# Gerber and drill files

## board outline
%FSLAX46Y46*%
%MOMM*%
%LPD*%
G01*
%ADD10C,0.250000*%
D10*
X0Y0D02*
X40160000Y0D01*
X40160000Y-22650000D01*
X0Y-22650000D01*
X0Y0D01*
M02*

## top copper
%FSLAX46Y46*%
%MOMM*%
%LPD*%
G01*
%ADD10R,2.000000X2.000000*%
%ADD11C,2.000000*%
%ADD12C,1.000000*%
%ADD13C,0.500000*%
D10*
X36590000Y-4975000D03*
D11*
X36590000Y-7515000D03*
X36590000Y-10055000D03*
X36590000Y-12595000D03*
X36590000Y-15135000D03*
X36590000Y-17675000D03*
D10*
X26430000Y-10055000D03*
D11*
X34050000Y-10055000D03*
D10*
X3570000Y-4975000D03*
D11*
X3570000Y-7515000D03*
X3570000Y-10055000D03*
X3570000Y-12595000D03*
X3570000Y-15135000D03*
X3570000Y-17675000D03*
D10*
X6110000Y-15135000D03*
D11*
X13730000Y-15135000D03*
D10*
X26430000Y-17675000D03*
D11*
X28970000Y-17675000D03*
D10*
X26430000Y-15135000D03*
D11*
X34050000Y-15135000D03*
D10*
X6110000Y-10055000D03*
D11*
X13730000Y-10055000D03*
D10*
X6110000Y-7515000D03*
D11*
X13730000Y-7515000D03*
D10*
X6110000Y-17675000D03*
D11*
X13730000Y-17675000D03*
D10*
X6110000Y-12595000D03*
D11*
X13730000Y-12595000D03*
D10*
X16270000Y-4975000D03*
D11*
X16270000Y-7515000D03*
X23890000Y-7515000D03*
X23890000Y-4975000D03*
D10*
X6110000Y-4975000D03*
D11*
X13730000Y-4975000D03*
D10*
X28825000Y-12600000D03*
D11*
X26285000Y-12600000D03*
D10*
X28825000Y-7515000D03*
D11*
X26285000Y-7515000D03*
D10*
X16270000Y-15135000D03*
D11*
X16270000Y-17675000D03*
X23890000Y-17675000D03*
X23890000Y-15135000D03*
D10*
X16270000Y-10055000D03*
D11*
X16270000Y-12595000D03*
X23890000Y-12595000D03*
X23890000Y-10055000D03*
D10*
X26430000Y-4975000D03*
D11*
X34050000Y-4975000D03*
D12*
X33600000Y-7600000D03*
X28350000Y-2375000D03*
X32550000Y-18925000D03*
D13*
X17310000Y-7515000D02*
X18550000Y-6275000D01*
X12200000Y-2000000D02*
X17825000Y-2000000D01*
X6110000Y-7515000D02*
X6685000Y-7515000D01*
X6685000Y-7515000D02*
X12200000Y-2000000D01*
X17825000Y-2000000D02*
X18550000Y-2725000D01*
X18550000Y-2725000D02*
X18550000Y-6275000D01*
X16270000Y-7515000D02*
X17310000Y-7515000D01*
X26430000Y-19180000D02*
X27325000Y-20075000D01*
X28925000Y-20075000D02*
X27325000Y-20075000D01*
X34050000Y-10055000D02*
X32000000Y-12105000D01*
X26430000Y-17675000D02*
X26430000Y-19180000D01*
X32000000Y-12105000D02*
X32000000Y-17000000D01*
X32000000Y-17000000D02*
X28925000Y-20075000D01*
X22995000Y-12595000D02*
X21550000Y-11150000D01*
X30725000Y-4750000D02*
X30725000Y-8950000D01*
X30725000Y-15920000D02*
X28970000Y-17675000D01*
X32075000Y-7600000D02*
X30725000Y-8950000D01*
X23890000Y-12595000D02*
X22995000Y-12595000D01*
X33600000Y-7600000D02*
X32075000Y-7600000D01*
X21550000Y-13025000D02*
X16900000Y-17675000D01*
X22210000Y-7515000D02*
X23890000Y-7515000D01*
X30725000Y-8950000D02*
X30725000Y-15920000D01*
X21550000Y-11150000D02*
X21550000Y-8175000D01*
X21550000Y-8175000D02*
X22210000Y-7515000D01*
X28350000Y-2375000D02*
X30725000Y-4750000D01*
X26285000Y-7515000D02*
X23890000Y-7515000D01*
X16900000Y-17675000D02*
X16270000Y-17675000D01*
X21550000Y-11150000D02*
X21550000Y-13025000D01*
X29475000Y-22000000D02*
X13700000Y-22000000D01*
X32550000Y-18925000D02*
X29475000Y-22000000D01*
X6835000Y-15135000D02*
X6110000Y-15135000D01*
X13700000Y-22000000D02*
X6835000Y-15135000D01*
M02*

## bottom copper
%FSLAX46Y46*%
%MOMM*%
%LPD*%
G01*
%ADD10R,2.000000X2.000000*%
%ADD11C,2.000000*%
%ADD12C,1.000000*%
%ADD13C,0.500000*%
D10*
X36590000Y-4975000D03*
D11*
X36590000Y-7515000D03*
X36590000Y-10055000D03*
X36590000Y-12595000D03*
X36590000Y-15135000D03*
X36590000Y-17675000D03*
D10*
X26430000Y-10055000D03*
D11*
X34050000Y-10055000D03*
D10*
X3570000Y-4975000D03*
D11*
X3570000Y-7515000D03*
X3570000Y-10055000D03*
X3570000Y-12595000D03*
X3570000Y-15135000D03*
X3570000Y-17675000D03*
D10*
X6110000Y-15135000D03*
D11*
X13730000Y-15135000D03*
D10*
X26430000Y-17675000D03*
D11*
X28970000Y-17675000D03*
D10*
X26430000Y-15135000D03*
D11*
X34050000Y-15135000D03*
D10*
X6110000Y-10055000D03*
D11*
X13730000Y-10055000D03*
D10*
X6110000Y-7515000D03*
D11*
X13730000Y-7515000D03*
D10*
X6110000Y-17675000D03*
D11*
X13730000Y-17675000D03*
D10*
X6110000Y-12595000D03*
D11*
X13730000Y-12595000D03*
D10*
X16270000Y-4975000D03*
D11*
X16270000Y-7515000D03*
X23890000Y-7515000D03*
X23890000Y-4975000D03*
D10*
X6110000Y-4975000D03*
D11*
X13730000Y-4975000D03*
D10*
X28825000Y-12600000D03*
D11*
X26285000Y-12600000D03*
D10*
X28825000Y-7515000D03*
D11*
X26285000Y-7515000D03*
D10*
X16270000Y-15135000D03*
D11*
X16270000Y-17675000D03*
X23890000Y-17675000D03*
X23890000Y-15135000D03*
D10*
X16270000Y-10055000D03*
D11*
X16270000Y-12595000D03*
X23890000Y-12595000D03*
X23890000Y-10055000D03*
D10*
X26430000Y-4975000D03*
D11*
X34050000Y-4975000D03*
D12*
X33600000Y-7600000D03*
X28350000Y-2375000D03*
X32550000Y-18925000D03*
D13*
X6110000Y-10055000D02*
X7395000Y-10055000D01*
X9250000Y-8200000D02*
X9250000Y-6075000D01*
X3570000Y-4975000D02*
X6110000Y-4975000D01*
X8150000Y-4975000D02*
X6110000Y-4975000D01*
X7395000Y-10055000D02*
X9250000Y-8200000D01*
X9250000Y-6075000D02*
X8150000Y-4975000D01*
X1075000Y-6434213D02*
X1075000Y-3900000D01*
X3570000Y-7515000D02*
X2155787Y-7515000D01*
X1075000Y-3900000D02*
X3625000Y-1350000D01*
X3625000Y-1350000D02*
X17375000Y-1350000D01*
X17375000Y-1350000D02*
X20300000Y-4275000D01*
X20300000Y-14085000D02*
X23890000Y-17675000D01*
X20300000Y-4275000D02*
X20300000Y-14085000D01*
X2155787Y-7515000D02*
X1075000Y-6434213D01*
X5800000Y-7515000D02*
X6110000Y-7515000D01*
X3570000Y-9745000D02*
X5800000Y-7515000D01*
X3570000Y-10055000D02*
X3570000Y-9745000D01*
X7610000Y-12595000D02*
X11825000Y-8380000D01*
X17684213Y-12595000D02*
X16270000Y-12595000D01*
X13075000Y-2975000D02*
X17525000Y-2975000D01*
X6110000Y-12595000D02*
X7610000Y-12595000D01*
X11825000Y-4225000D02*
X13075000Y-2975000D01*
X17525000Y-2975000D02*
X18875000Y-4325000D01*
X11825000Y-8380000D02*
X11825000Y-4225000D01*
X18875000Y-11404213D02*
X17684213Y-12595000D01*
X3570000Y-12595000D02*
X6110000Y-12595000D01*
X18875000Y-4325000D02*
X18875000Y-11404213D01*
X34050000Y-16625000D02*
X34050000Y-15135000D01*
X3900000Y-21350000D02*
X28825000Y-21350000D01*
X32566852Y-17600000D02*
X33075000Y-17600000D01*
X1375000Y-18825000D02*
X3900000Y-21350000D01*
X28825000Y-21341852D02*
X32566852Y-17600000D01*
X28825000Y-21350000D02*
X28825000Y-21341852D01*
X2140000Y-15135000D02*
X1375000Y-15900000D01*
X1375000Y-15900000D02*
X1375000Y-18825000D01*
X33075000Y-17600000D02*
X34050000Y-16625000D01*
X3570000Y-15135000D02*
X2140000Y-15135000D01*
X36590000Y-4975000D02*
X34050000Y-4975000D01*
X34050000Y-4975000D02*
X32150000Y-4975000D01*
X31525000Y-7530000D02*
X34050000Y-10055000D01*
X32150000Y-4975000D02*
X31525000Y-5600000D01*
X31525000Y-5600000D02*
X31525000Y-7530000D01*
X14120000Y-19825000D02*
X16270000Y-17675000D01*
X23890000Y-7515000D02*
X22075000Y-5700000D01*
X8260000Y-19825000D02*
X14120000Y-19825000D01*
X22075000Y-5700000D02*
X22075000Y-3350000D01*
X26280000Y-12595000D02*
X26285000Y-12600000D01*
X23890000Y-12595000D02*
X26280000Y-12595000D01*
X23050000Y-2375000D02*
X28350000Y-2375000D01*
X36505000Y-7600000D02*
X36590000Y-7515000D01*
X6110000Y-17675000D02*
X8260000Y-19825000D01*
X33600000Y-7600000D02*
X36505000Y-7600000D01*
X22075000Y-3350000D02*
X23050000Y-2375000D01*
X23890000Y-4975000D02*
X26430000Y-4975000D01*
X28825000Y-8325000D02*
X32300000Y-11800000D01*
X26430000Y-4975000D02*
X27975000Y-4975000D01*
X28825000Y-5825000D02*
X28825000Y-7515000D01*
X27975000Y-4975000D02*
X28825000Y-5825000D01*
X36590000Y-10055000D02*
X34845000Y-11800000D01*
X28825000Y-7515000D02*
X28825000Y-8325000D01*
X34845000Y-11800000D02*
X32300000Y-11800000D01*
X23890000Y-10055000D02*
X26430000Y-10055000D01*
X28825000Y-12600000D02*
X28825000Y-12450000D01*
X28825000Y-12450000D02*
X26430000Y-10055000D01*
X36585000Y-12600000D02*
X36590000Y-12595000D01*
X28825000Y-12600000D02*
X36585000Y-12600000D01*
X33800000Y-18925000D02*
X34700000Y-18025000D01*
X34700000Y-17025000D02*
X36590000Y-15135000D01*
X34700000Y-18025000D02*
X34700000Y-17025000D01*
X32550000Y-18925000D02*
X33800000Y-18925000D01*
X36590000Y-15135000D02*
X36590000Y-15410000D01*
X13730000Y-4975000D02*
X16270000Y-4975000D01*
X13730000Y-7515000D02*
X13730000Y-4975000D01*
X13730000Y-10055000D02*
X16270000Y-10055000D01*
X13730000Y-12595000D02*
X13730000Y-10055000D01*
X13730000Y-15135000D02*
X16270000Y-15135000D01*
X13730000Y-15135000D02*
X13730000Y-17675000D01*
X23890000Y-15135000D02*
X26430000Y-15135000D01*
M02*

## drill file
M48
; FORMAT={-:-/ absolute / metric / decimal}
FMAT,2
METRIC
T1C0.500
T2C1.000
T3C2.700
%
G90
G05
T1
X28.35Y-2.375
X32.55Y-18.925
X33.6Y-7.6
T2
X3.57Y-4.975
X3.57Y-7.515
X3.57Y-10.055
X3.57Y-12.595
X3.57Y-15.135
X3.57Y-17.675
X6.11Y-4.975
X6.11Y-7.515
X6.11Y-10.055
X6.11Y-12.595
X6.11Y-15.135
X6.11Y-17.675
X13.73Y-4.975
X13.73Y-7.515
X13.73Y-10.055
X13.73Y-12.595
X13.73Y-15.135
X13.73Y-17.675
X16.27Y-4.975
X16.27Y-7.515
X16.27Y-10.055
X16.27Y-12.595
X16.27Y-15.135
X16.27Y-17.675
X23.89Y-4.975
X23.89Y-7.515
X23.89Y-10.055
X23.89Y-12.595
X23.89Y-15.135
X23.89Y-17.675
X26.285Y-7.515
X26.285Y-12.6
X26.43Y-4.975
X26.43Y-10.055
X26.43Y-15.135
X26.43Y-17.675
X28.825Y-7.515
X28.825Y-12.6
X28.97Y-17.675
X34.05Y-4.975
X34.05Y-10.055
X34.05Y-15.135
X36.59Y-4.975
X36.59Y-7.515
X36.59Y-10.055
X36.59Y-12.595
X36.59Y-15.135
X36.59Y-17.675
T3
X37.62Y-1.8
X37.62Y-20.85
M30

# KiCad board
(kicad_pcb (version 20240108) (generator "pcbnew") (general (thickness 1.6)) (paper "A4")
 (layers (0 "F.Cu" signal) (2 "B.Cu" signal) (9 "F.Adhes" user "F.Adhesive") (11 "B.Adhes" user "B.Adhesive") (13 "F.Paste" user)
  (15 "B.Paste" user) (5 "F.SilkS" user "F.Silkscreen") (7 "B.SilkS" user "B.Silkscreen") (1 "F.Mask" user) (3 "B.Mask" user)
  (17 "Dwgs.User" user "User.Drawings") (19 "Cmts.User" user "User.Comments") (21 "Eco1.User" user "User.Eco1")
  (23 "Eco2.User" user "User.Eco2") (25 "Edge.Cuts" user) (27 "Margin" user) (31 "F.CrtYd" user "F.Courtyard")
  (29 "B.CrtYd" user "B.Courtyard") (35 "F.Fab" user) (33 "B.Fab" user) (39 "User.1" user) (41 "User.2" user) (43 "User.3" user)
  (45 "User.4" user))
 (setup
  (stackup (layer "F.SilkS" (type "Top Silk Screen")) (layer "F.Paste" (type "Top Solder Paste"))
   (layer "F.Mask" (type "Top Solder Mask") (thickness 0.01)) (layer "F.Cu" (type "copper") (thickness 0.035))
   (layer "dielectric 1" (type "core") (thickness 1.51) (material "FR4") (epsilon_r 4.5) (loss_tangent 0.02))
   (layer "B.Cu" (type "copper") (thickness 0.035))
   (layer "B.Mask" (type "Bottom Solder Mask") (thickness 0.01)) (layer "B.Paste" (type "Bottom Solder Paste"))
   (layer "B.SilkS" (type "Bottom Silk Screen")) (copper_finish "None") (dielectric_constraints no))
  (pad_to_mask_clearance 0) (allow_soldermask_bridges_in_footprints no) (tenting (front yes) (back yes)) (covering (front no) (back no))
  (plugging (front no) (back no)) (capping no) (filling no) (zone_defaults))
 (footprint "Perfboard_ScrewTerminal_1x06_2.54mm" (layer "F.Cu") (at 36.59 4.975)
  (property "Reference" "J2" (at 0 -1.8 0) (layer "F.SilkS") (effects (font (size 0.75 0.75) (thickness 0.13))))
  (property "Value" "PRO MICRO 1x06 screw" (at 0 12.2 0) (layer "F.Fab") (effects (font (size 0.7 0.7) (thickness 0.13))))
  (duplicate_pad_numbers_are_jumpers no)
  (pad "1" thru_hole rect (at 0 0) (size 2 2) (drill 1) (layers "*.Cu" "*.Mask") (remove_unused_layers no) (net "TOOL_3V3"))
  (pad "2" thru_hole circle (at 0 2.54) (size 2 2) (drill 1) (layers "*.Cu" "*.Mask") (remove_unused_layers no) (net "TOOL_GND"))
  (pad "3" thru_hole circle (at 0 5.08) (size 2 2) (drill 1) (layers "*.Cu" "*.Mask") (remove_unused_layers no) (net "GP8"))
  (pad "4" thru_hole circle (at 0 7.62) (size 2 2) (drill 1) (layers "*.Cu" "*.Mask") (remove_unused_layers no) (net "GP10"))
  (pad "5" thru_hole circle (at 0 10.16) (size 2 2) (drill 1) (layers "*.Cu" "*.Mask") (remove_unused_layers no) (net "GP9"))
  (pad "6" thru_hole circle (at 0 12.7) (size 2 2) (drill 1) (layers "*.Cu" "*.Mask") (remove_unused_layers no)))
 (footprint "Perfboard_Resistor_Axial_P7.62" (layer "F.Cu") (at 26.43 10.055)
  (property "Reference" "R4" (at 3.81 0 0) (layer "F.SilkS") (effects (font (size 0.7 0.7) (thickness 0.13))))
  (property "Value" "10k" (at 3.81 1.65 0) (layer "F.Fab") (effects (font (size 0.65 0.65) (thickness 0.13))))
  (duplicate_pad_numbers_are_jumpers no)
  (pad "1" thru_hole rect (at 0 0) (size 2 2) (drill 1) (layers "*.Cu" "*.Mask") (remove_unused_layers no) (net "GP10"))
  (pad "2" thru_hole circle (at 7.62 0) (size 2 2) (drill 1) (layers "*.Cu" "*.Mask") (remove_unused_layers no) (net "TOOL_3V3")))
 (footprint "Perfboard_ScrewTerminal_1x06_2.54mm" (layer "F.Cu") (at 3.57 4.975)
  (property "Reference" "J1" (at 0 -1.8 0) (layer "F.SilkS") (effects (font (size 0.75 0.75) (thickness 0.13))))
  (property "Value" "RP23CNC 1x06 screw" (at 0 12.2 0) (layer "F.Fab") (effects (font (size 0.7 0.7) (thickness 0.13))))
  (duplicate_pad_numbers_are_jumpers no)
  (pad "1" thru_hole rect (at 0 0) (size 2 2) (drill 1) (layers "*.Cu" "*.Mask") (remove_unused_layers no) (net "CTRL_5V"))
  (pad "2" thru_hole circle (at 0 2.54) (size 2 2) (drill 1) (layers "*.Cu" "*.Mask") (remove_unused_layers no) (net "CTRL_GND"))
  (pad "3" thru_hole circle (at 0 5.08) (size 2 2) (drill 1) (layers "*.Cu" "*.Mask") (remove_unused_layers no) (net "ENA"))
  (pad "4" thru_hole circle (at 0 7.62) (size 2 2) (drill 1) (layers "*.Cu" "*.Mask") (remove_unused_layers no) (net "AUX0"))
  (pad "5" thru_hole circle (at 0 10.16) (size 2 2) (drill 1) (layers "*.Cu" "*.Mask") (remove_unused_layers no) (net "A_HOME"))
  (pad "6" thru_hole circle (at 0 12.7) (size 2 2) (drill 1) (layers "*.Cu" "*.Mask") (remove_unused_layers no)))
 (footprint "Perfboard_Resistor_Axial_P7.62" (layer "F.Cu") (at 6.11 15.135)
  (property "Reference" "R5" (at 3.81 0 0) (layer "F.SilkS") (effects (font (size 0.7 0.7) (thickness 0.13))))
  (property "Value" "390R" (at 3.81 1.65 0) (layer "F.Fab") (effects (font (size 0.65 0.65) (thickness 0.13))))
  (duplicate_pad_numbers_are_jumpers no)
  (pad "1" thru_hole rect (at 0 0) (size 2 2) (drill 1) (layers "*.Cu" "*.Mask") (remove_unused_layers no) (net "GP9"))
  (pad "2" thru_hole circle (at 7.62 0) (size 2 2) (drill 1) (layers "*.Cu" "*.Mask") (remove_unused_layers no) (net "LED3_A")))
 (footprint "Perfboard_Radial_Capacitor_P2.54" (layer "F.Cu") (at 26.43 17.675)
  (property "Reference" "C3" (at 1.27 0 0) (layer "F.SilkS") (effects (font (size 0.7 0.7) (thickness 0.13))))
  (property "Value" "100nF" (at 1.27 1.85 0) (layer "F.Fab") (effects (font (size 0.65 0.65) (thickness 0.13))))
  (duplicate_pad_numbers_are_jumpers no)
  (pad "1" thru_hole rect (at 0 0) (size 2 2) (drill 1) (layers "*.Cu" "*.Mask") (remove_unused_layers no) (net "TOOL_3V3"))
  (pad "2" thru_hole circle (at 2.54 0) (size 2 2) (drill 1) (layers "*.Cu" "*.Mask") (remove_unused_layers no) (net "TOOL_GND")))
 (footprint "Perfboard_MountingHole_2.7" (layer "F.Cu") (at 37.62 1.8)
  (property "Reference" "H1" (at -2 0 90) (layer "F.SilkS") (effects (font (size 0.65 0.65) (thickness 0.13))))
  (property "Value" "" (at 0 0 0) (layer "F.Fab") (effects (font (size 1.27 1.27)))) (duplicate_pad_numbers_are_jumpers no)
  (pad "" np_thru_hole circle (at 0 0) (size 2.7 2.7) (drill 2.7) (layers "*.Cu" "*.Mask")))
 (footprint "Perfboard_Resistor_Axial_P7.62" (layer "F.Cu") (at 26.43 15.135)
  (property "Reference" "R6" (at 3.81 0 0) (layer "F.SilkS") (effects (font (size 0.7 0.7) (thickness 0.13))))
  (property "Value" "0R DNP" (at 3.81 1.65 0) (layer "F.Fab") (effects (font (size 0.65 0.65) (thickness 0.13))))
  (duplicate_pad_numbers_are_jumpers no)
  (pad "1" thru_hole rect (at 0 0) (size 2 2) (drill 1) (layers "*.Cu" "*.Mask") (remove_unused_layers no) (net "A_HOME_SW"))
  (pad "2" thru_hole circle (at 7.62 0) (size 2 2) (drill 1) (layers "*.Cu" "*.Mask") (remove_unused_layers no) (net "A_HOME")))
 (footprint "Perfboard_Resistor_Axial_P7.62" (layer "F.Cu") (at 6.11 10.055)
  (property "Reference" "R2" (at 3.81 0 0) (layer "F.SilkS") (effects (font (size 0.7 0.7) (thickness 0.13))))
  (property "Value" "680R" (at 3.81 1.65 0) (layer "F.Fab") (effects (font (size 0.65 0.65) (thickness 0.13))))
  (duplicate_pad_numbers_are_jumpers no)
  (pad "1" thru_hole rect (at 0 0) (size 2 2) (drill 1) (layers "*.Cu" "*.Mask") (remove_unused_layers no) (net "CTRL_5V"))
  (pad "2" thru_hole circle (at 7.62 0) (size 2 2) (drill 1) (layers "*.Cu" "*.Mask") (remove_unused_layers no) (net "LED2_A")))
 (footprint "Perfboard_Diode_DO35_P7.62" (layer "F.Cu") (at 6.11 7.515)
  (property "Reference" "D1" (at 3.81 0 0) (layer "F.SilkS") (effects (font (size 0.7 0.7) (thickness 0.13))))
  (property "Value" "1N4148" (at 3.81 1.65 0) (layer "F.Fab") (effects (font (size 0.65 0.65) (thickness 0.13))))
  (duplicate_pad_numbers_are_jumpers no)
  (pad "1" thru_hole rect (at 0 0) (size 2 2) (drill 1) (layers "*.Cu" "*.Mask") (remove_unused_layers no) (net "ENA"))
  (pad "2" thru_hole circle (at 7.62 0) (size 2 2) (drill 1) (layers "*.Cu" "*.Mask") (remove_unused_layers no) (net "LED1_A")))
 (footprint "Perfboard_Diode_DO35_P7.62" (layer "F.Cu") (at 6.11 17.675)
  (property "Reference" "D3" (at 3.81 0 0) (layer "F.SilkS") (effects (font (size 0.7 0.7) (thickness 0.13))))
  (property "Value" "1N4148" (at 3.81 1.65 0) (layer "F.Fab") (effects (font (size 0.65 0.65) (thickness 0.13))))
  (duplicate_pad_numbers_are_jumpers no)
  (pad "1" thru_hole rect (at 0 0) (size 2 2) (drill 1) (layers "*.Cu" "*.Mask") (remove_unused_layers no) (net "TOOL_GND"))
  (pad "2" thru_hole circle (at 7.62 0) (size 2 2) (drill 1) (layers "*.Cu" "*.Mask") (remove_unused_layers no) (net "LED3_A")))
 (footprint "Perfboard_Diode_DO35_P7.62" (layer "F.Cu") (at 6.11 12.595)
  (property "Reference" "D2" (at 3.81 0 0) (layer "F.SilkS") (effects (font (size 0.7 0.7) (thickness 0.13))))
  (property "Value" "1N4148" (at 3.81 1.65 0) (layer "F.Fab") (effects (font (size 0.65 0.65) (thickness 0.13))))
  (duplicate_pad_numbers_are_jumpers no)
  (pad "1" thru_hole rect (at 0 0) (size 2 2) (drill 1) (layers "*.Cu" "*.Mask") (remove_unused_layers no) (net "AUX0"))
  (pad "2" thru_hole circle (at 7.62 0) (size 2 2) (drill 1) (layers "*.Cu" "*.Mask") (remove_unused_layers no) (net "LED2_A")))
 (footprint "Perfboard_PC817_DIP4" (layer "F.Cu") (at 16.27 4.975)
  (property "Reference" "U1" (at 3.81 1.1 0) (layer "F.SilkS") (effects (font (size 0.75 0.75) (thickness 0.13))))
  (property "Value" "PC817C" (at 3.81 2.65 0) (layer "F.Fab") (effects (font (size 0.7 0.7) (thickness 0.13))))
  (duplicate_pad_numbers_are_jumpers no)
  (pad "1" thru_hole rect (at 0 0) (size 2 2) (drill 1) (layers "*.Cu" "*.Mask") (remove_unused_layers no) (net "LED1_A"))
  (pad "2" thru_hole circle (at 0 2.54) (size 2 2) (drill 1) (layers "*.Cu" "*.Mask") (remove_unused_layers no) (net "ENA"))
  (pad "3" thru_hole circle (at 7.62 2.54) (size 2 2) (drill 1) (layers "*.Cu" "*.Mask") (remove_unused_layers no) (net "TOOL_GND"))
  (pad "4" thru_hole circle (at 7.62 0) (size 2 2) (drill 1) (layers "*.Cu" "*.Mask") (remove_unused_layers no) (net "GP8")))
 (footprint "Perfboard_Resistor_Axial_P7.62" (layer "F.Cu") (at 6.11 4.975)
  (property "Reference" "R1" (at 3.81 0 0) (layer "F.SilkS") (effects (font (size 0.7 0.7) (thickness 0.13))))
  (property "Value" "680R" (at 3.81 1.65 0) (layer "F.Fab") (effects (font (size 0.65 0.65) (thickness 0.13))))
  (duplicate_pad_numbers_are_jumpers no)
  (pad "1" thru_hole rect (at 0 0) (size 2 2) (drill 1) (layers "*.Cu" "*.Mask") (remove_unused_layers no) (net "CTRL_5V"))
  (pad "2" thru_hole circle (at 7.62 0) (size 2 2) (drill 1) (layers "*.Cu" "*.Mask") (remove_unused_layers no) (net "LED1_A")))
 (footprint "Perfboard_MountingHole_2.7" (layer "F.Cu") (at 37.62 20.85)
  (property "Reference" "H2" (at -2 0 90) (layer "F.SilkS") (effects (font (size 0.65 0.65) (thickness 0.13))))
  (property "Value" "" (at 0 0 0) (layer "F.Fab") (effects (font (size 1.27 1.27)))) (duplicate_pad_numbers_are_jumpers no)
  (pad "" np_thru_hole circle (at 0 0) (size 2.7 2.7) (drill 2.7) (layers "*.Cu" "*.Mask")))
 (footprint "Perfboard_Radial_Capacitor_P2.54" (layer "F.Cu") (at 28.825 12.6 180)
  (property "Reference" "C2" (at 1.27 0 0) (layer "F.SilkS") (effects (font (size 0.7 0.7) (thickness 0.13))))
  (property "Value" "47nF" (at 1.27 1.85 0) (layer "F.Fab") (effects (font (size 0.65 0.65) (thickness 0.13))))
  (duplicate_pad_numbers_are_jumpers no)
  (pad "1" thru_hole rect (at 0 0 180) (size 2 2) (drill 1) (layers "*.Cu" "*.Mask") (remove_unused_layers no) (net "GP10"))
  (pad "2" thru_hole circle (at 2.54 0 180) (size 2 2) (drill 1) (layers "*.Cu" "*.Mask") (remove_unused_layers no) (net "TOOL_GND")))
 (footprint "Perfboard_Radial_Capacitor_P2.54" (layer "F.Cu") (at 28.825 7.515 180)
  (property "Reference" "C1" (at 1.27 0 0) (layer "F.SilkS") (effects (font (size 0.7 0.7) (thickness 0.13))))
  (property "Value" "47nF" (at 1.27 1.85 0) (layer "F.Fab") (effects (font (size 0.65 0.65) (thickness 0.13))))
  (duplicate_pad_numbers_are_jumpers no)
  (pad "1" thru_hole rect (at 0 0 180) (size 2 2) (drill 1) (layers "*.Cu" "*.Mask") (remove_unused_layers no) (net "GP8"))
  (pad "2" thru_hole circle (at 2.54 0 180) (size 2 2) (drill 1) (layers "*.Cu" "*.Mask") (remove_unused_layers no) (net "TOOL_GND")))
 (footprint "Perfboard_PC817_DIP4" (layer "F.Cu") (at 16.27 15.135)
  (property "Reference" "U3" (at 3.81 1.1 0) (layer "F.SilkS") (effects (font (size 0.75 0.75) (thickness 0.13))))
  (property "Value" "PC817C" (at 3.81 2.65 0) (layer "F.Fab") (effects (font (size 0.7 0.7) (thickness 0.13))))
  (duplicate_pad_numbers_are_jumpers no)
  (pad "1" thru_hole rect (at 0 0) (size 2 2) (drill 1) (layers "*.Cu" "*.Mask") (remove_unused_layers no) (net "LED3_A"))
  (pad "2" thru_hole circle (at 0 2.54) (size 2 2) (drill 1) (layers "*.Cu" "*.Mask") (remove_unused_layers no) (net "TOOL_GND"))
  (pad "3" thru_hole circle (at 7.62 2.54) (size 2 2) (drill 1) (layers "*.Cu" "*.Mask") (remove_unused_layers no) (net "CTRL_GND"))
  (pad "4" thru_hole circle (at 7.62 0) (size 2 2) (drill 1) (layers "*.Cu" "*.Mask") (remove_unused_layers no) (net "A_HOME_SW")))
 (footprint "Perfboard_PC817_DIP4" (layer "F.Cu") (at 16.27 10.055)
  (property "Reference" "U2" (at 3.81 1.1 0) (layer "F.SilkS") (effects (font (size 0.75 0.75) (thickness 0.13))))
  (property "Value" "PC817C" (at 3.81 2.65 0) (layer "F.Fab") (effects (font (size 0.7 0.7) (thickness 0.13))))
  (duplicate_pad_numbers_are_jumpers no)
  (pad "1" thru_hole rect (at 0 0) (size 2 2) (drill 1) (layers "*.Cu" "*.Mask") (remove_unused_layers no) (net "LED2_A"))
  (pad "2" thru_hole circle (at 0 2.54) (size 2 2) (drill 1) (layers "*.Cu" "*.Mask") (remove_unused_layers no) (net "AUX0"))
  (pad "3" thru_hole circle (at 7.62 2.54) (size 2 2) (drill 1) (layers "*.Cu" "*.Mask") (remove_unused_layers no) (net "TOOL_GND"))
  (pad "4" thru_hole circle (at 7.62 0) (size 2 2) (drill 1) (layers "*.Cu" "*.Mask") (remove_unused_layers no) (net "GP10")))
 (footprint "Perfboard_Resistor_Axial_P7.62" (layer "F.Cu") (at 26.43 4.975)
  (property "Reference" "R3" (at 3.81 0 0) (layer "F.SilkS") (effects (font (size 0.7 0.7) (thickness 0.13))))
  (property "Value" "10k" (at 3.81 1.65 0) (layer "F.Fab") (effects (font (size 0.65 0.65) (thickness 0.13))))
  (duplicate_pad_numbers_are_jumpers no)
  (pad "1" thru_hole rect (at 0 0) (size 2 2) (drill 1) (layers "*.Cu" "*.Mask") (remove_unused_layers no) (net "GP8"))
  (pad "2" thru_hole circle (at 7.62 0) (size 2 2) (drill 1) (layers "*.Cu" "*.Mask") (remove_unused_layers no) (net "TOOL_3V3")))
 (gr_rect (start 0 0) (end 40.16 22.65) (stroke (width 0.25) (type default)) (fill no) (layer "Edge.Cuts"))
 (segment (start 6.11 10.055) (end 7.395 10.055) (width 0.5) (layer "B.Cu") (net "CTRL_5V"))
 (segment (start 9.25 8.2) (end 9.25 6.075) (width 0.5) (layer "B.Cu") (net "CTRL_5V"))
 (segment (start 3.57 4.975) (end 6.11 4.975) (width 0.5) (layer "B.Cu") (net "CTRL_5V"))
 (segment (start 8.15 4.975) (end 6.11 4.975) (width 0.5) (layer "B.Cu") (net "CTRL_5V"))
 (segment (start 7.395 10.055) (end 9.25 8.2) (width 0.5) (layer "B.Cu") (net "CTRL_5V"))
 (segment (start 9.25 6.075) (end 8.15 4.975) (width 0.5) (layer "B.Cu") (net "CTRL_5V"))
 (segment (start 1.075 6.434213) (end 1.075 3.9) (width 0.5) (layer "B.Cu") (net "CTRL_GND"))
 (segment (start 3.57 7.515) (end 2.155787 7.515) (width 0.5) (layer "B.Cu") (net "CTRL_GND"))
 (segment (start 1.075 3.9) (end 3.625 1.35) (width 0.5) (layer "B.Cu") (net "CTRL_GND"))
 (segment (start 3.625 1.35) (end 17.375 1.35) (width 0.5) (layer "B.Cu") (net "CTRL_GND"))
 (segment (start 17.375 1.35) (end 20.3 4.275) (width 0.5) (layer "B.Cu") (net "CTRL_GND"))
 (segment (start 20.3 14.085) (end 23.89 17.675) (width 0.5) (layer "B.Cu") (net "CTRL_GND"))
 (segment (start 20.3 4.275) (end 20.3 14.085) (width 0.5) (layer "B.Cu") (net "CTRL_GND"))
 (segment (start 2.155787 7.515) (end 1.075 6.434213) (width 0.5) (layer "B.Cu") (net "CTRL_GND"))
 (segment (start 17.31 7.515) (end 18.55 6.275) (width 0.5) (layer "F.Cu") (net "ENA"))
 (segment (start 12.2 2) (end 17.825 2) (width 0.5) (layer "F.Cu") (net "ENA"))
 (segment (start 6.11 7.515) (end 6.685 7.515) (width 0.5) (layer "F.Cu") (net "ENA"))
 (segment (start 6.685 7.515) (end 12.2 2) (width 0.5) (layer "F.Cu") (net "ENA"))
 (segment (start 17.825 2) (end 18.55 2.725) (width 0.5) (layer "F.Cu") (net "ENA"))
 (segment (start 18.55 2.725) (end 18.55 6.275) (width 0.5) (layer "F.Cu") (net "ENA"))
 (segment (start 16.27 7.515) (end 17.31 7.515) (width 0.5) (layer "F.Cu") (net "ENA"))
 (segment (start 5.8 7.515) (end 6.11 7.515) (width 0.5) (layer "B.Cu") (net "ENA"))
 (segment (start 3.57 9.745) (end 5.8 7.515) (width 0.5) (layer "B.Cu") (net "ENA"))
 (segment (start 3.57 10.055) (end 3.57 9.745) (width 0.5) (layer "B.Cu") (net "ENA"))
 (segment (start 7.61 12.595) (end 11.825 8.38) (width 0.5) (layer "B.Cu") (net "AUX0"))
 (segment (start 17.684213 12.595) (end 16.27 12.595) (width 0.5) (layer "B.Cu") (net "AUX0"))
 (segment (start 13.075 2.975) (end 17.525 2.975) (width 0.5) (layer "B.Cu") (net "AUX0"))
 (segment (start 6.11 12.595) (end 7.61 12.595) (width 0.5) (layer "B.Cu") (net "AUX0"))
 (segment (start 11.825 4.225) (end 13.075 2.975) (width 0.5) (layer "B.Cu") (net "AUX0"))
 (segment (start 17.525 2.975) (end 18.875 4.325) (width 0.5) (layer "B.Cu") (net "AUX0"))
 (segment (start 11.825 8.38) (end 11.825 4.225) (width 0.5) (layer "B.Cu") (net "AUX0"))
 (segment (start 18.875 11.404213) (end 17.684213 12.595) (width 0.5) (layer "B.Cu") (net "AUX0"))
 (segment (start 3.57 12.595) (end 6.11 12.595) (width 0.5) (layer "B.Cu") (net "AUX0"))
 (segment (start 18.875 4.325) (end 18.875 11.404213) (width 0.5) (layer "B.Cu") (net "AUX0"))
 (segment (start 34.05 16.625) (end 34.05 15.135) (width 0.5) (layer "B.Cu") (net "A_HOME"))
 (segment (start 3.9 21.35) (end 28.825 21.35) (width 0.5) (layer "B.Cu") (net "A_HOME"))
 (segment (start 32.566852 17.6) (end 33.075 17.6) (width 0.5) (layer "B.Cu") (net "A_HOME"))
 (segment (start 1.375 18.825) (end 3.9 21.35) (width 0.5) (layer "B.Cu") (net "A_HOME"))
 (segment (start 28.825 21.341852) (end 32.566852 17.6) (width 0.5) (layer "B.Cu") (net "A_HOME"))
 (segment (start 28.825 21.35) (end 28.825 21.341852) (width 0.5) (layer "B.Cu") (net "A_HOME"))
 (segment (start 2.14 15.135) (end 1.375 15.9) (width 0.5) (layer "B.Cu") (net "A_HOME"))
 (segment (start 1.375 15.9) (end 1.375 18.825) (width 0.5) (layer "B.Cu") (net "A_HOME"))
 (segment (start 33.075 17.6) (end 34.05 16.625) (width 0.5) (layer "B.Cu") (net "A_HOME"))
 (segment (start 3.57 15.135) (end 2.14 15.135) (width 0.5) (layer "B.Cu") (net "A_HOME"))
 (segment (start 26.43 19.18) (end 27.325 20.075) (width 0.5) (layer "F.Cu") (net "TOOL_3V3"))
 (segment (start 28.925 20.075) (end 27.325 20.075) (width 0.5) (layer "F.Cu") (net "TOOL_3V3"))
 (segment (start 34.05 10.055) (end 32 12.105) (width 0.5) (layer "F.Cu") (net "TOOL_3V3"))
 (segment (start 26.43 17.675) (end 26.43 19.18) (width 0.5) (layer "F.Cu") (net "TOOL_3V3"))
 (segment (start 32 12.105) (end 32 17) (width 0.5) (layer "F.Cu") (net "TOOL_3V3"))
 (segment (start 32 17) (end 28.925 20.075) (width 0.5) (layer "F.Cu") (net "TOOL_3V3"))
 (segment (start 36.59 4.975) (end 34.05 4.975) (width 0.5) (layer "B.Cu") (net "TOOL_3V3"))
 (segment (start 34.05 4.975) (end 32.15 4.975) (width 0.5) (layer "B.Cu") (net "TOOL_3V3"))
 (segment (start 31.525 7.53) (end 34.05 10.055) (width 0.5) (layer "B.Cu") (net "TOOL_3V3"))
 (segment (start 32.15 4.975) (end 31.525 5.6) (width 0.5) (layer "B.Cu") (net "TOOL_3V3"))
 (segment (start 31.525 5.6) (end 31.525 7.53) (width 0.5) (layer "B.Cu") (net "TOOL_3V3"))
 (segment (start 22.995 12.595) (end 21.55 11.15) (width 0.5) (layer "F.Cu") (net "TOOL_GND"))
 (segment (start 30.725 4.75) (end 30.725 8.95) (width 0.5) (layer "F.Cu") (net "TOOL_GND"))
 (segment (start 30.725 15.92) (end 28.97 17.675) (width 0.5) (layer "F.Cu") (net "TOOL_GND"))
 (segment (start 32.075 7.6) (end 30.725 8.95) (width 0.5) (layer "F.Cu") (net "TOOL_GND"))
 (segment (start 23.89 12.595) (end 22.995 12.595) (width 0.5) (layer "F.Cu") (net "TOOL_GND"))
 (segment (start 33.6 7.6) (end 32.075 7.6) (width 0.5) (layer "F.Cu") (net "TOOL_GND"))
 (segment (start 21.55 13.025) (end 16.9 17.675) (width 0.5) (layer "F.Cu") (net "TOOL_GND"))
 (segment (start 22.21 7.515) (end 23.89 7.515) (width 0.5) (layer "F.Cu") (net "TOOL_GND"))
 (segment (start 30.725 8.95) (end 30.725 15.92) (width 0.5) (layer "F.Cu") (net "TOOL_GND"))
 (segment (start 21.55 11.15) (end 21.55 8.175) (width 0.5) (layer "F.Cu") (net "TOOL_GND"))
 (segment (start 21.55 8.175) (end 22.21 7.515) (width 0.5) (layer "F.Cu") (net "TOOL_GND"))
 (segment (start 28.35 2.375) (end 30.725 4.75) (width 0.5) (layer "F.Cu") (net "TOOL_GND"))
 (segment (start 26.285 7.515) (end 23.89 7.515) (width 0.5) (layer "F.Cu") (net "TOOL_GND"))
 (segment (start 16.9 17.675) (end 16.27 17.675) (width 0.5) (layer "F.Cu") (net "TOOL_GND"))
 (segment (start 21.55 11.15) (end 21.55 13.025) (width 0.5) (layer "F.Cu") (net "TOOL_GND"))
 (via (at 33.6 7.6) (size 1) (drill 0.5) (layers "F.Cu" "B.Cu") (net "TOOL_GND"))
 (via (at 28.35 2.375) (size 1) (drill 0.5) (layers "F.Cu" "B.Cu") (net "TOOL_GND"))
 (segment (start 14.12 19.825) (end 16.27 17.675) (width 0.5) (layer "B.Cu") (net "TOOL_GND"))
 (segment (start 23.89 7.515) (end 22.075 5.7) (width 0.5) (layer "B.Cu") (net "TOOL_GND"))
 (segment (start 8.26 19.825) (end 14.12 19.825) (width 0.5) (layer "B.Cu") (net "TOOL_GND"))
 (segment (start 22.075 5.7) (end 22.075 3.35) (width 0.5) (layer "B.Cu") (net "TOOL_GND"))
 (segment (start 26.28 12.595) (end 26.285 12.6) (width 0.5) (layer "B.Cu") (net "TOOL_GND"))
 (segment (start 23.89 12.595) (end 26.28 12.595) (width 0.5) (layer "B.Cu") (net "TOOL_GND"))
 (segment (start 23.05 2.375) (end 28.35 2.375) (width 0.5) (layer "B.Cu") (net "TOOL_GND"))
 (segment (start 36.505 7.6) (end 36.59 7.515) (width 0.5) (layer "B.Cu") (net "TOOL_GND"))
 (segment (start 6.11 17.675) (end 8.26 19.825) (width 0.5) (layer "B.Cu") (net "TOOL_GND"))
 (segment (start 33.6 7.6) (end 36.505 7.6) (width 0.5) (layer "B.Cu") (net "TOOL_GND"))
 (segment (start 22.075 3.35) (end 23.05 2.375) (width 0.5) (layer "B.Cu") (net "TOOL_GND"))
 (segment (start 23.89 4.975) (end 26.43 4.975) (width 0.5) (layer "B.Cu") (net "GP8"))
 (segment (start 28.825 8.325) (end 32.3 11.8) (width 0.5) (layer "B.Cu") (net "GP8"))
 (segment (start 26.43 4.975) (end 27.975 4.975) (width 0.5) (layer "B.Cu") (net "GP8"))
 (segment (start 28.825 5.825) (end 28.825 7.515) (width 0.5) (layer "B.Cu") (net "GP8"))
 (segment (start 27.975 4.975) (end 28.825 5.825) (width 0.5) (layer "B.Cu") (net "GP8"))
 (segment (start 36.59 10.055) (end 34.845 11.8) (width 0.5) (layer "B.Cu") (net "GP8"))
 (segment (start 28.825 7.515) (end 28.825 8.325) (width 0.5) (layer "B.Cu") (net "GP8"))
 (segment (start 34.845 11.8) (end 32.3 11.8) (width 0.5) (layer "B.Cu") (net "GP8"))
 (segment (start 23.89 10.055) (end 26.43 10.055) (width 0.5) (layer "B.Cu") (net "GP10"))
 (segment (start 28.825 12.6) (end 28.825 12.45) (width 0.5) (layer "B.Cu") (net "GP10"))
 (segment (start 28.825 12.45) (end 26.43 10.055) (width 0.5) (layer "B.Cu") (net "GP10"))
 (segment (start 36.585 12.6) (end 36.59 12.595) (width 0.5) (layer "B.Cu") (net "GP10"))
 (segment (start 28.825 12.6) (end 36.585 12.6) (width 0.5) (layer "B.Cu") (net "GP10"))
 (segment (start 29.475 22) (end 13.7 22) (width 0.5) (layer "F.Cu") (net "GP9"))
 (segment (start 32.55 18.925) (end 29.475 22) (width 0.5) (layer "F.Cu") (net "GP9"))
 (segment (start 6.835 15.135) (end 6.11 15.135) (width 0.5) (layer "F.Cu") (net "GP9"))
 (segment (start 13.7 22) (end 6.835 15.135) (width 0.5) (layer "F.Cu") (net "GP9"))
 (via (at 32.55 18.925) (size 1) (drill 0.5) (layers "F.Cu" "B.Cu") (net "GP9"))
 (segment (start 33.8 18.925) (end 34.7 18.025) (width 0.5) (layer "B.Cu") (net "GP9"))
 (segment (start 34.7 17.025) (end 36.59 15.135) (width 0.5) (layer "B.Cu") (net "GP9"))
 (segment (start 34.7 18.025) (end 34.7 17.025) (width 0.5) (layer "B.Cu") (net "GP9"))
 (segment (start 32.55 18.925) (end 33.8 18.925) (width 0.5) (layer "B.Cu") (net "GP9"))
 (segment (start 36.59 15.135) (end 36.59 15.41) (width 0.5) (layer "B.Cu") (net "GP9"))
 (segment (start 13.73 4.975) (end 16.27 4.975) (width 0.5) (layer "B.Cu") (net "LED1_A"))
 (segment (start 13.73 7.515) (end 13.73 4.975) (width 0.5) (layer "B.Cu") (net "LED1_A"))
 (segment (start 13.73 10.055) (end 16.27 10.055) (width 0.5) (layer "B.Cu") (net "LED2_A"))
 (segment (start 13.73 12.595) (end 13.73 10.055) (width 0.5) (layer "B.Cu") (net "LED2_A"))
 (segment (start 13.73 15.135) (end 16.27 15.135) (width 0.5) (layer "B.Cu") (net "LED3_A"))
 (segment (start 13.73 15.135) (end 13.73 17.675) (width 0.5) (layer "B.Cu") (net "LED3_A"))
 (segment (start 23.89 15.135) (end 26.43 15.135) (width 0.5) (layer "B.Cu") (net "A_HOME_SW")))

